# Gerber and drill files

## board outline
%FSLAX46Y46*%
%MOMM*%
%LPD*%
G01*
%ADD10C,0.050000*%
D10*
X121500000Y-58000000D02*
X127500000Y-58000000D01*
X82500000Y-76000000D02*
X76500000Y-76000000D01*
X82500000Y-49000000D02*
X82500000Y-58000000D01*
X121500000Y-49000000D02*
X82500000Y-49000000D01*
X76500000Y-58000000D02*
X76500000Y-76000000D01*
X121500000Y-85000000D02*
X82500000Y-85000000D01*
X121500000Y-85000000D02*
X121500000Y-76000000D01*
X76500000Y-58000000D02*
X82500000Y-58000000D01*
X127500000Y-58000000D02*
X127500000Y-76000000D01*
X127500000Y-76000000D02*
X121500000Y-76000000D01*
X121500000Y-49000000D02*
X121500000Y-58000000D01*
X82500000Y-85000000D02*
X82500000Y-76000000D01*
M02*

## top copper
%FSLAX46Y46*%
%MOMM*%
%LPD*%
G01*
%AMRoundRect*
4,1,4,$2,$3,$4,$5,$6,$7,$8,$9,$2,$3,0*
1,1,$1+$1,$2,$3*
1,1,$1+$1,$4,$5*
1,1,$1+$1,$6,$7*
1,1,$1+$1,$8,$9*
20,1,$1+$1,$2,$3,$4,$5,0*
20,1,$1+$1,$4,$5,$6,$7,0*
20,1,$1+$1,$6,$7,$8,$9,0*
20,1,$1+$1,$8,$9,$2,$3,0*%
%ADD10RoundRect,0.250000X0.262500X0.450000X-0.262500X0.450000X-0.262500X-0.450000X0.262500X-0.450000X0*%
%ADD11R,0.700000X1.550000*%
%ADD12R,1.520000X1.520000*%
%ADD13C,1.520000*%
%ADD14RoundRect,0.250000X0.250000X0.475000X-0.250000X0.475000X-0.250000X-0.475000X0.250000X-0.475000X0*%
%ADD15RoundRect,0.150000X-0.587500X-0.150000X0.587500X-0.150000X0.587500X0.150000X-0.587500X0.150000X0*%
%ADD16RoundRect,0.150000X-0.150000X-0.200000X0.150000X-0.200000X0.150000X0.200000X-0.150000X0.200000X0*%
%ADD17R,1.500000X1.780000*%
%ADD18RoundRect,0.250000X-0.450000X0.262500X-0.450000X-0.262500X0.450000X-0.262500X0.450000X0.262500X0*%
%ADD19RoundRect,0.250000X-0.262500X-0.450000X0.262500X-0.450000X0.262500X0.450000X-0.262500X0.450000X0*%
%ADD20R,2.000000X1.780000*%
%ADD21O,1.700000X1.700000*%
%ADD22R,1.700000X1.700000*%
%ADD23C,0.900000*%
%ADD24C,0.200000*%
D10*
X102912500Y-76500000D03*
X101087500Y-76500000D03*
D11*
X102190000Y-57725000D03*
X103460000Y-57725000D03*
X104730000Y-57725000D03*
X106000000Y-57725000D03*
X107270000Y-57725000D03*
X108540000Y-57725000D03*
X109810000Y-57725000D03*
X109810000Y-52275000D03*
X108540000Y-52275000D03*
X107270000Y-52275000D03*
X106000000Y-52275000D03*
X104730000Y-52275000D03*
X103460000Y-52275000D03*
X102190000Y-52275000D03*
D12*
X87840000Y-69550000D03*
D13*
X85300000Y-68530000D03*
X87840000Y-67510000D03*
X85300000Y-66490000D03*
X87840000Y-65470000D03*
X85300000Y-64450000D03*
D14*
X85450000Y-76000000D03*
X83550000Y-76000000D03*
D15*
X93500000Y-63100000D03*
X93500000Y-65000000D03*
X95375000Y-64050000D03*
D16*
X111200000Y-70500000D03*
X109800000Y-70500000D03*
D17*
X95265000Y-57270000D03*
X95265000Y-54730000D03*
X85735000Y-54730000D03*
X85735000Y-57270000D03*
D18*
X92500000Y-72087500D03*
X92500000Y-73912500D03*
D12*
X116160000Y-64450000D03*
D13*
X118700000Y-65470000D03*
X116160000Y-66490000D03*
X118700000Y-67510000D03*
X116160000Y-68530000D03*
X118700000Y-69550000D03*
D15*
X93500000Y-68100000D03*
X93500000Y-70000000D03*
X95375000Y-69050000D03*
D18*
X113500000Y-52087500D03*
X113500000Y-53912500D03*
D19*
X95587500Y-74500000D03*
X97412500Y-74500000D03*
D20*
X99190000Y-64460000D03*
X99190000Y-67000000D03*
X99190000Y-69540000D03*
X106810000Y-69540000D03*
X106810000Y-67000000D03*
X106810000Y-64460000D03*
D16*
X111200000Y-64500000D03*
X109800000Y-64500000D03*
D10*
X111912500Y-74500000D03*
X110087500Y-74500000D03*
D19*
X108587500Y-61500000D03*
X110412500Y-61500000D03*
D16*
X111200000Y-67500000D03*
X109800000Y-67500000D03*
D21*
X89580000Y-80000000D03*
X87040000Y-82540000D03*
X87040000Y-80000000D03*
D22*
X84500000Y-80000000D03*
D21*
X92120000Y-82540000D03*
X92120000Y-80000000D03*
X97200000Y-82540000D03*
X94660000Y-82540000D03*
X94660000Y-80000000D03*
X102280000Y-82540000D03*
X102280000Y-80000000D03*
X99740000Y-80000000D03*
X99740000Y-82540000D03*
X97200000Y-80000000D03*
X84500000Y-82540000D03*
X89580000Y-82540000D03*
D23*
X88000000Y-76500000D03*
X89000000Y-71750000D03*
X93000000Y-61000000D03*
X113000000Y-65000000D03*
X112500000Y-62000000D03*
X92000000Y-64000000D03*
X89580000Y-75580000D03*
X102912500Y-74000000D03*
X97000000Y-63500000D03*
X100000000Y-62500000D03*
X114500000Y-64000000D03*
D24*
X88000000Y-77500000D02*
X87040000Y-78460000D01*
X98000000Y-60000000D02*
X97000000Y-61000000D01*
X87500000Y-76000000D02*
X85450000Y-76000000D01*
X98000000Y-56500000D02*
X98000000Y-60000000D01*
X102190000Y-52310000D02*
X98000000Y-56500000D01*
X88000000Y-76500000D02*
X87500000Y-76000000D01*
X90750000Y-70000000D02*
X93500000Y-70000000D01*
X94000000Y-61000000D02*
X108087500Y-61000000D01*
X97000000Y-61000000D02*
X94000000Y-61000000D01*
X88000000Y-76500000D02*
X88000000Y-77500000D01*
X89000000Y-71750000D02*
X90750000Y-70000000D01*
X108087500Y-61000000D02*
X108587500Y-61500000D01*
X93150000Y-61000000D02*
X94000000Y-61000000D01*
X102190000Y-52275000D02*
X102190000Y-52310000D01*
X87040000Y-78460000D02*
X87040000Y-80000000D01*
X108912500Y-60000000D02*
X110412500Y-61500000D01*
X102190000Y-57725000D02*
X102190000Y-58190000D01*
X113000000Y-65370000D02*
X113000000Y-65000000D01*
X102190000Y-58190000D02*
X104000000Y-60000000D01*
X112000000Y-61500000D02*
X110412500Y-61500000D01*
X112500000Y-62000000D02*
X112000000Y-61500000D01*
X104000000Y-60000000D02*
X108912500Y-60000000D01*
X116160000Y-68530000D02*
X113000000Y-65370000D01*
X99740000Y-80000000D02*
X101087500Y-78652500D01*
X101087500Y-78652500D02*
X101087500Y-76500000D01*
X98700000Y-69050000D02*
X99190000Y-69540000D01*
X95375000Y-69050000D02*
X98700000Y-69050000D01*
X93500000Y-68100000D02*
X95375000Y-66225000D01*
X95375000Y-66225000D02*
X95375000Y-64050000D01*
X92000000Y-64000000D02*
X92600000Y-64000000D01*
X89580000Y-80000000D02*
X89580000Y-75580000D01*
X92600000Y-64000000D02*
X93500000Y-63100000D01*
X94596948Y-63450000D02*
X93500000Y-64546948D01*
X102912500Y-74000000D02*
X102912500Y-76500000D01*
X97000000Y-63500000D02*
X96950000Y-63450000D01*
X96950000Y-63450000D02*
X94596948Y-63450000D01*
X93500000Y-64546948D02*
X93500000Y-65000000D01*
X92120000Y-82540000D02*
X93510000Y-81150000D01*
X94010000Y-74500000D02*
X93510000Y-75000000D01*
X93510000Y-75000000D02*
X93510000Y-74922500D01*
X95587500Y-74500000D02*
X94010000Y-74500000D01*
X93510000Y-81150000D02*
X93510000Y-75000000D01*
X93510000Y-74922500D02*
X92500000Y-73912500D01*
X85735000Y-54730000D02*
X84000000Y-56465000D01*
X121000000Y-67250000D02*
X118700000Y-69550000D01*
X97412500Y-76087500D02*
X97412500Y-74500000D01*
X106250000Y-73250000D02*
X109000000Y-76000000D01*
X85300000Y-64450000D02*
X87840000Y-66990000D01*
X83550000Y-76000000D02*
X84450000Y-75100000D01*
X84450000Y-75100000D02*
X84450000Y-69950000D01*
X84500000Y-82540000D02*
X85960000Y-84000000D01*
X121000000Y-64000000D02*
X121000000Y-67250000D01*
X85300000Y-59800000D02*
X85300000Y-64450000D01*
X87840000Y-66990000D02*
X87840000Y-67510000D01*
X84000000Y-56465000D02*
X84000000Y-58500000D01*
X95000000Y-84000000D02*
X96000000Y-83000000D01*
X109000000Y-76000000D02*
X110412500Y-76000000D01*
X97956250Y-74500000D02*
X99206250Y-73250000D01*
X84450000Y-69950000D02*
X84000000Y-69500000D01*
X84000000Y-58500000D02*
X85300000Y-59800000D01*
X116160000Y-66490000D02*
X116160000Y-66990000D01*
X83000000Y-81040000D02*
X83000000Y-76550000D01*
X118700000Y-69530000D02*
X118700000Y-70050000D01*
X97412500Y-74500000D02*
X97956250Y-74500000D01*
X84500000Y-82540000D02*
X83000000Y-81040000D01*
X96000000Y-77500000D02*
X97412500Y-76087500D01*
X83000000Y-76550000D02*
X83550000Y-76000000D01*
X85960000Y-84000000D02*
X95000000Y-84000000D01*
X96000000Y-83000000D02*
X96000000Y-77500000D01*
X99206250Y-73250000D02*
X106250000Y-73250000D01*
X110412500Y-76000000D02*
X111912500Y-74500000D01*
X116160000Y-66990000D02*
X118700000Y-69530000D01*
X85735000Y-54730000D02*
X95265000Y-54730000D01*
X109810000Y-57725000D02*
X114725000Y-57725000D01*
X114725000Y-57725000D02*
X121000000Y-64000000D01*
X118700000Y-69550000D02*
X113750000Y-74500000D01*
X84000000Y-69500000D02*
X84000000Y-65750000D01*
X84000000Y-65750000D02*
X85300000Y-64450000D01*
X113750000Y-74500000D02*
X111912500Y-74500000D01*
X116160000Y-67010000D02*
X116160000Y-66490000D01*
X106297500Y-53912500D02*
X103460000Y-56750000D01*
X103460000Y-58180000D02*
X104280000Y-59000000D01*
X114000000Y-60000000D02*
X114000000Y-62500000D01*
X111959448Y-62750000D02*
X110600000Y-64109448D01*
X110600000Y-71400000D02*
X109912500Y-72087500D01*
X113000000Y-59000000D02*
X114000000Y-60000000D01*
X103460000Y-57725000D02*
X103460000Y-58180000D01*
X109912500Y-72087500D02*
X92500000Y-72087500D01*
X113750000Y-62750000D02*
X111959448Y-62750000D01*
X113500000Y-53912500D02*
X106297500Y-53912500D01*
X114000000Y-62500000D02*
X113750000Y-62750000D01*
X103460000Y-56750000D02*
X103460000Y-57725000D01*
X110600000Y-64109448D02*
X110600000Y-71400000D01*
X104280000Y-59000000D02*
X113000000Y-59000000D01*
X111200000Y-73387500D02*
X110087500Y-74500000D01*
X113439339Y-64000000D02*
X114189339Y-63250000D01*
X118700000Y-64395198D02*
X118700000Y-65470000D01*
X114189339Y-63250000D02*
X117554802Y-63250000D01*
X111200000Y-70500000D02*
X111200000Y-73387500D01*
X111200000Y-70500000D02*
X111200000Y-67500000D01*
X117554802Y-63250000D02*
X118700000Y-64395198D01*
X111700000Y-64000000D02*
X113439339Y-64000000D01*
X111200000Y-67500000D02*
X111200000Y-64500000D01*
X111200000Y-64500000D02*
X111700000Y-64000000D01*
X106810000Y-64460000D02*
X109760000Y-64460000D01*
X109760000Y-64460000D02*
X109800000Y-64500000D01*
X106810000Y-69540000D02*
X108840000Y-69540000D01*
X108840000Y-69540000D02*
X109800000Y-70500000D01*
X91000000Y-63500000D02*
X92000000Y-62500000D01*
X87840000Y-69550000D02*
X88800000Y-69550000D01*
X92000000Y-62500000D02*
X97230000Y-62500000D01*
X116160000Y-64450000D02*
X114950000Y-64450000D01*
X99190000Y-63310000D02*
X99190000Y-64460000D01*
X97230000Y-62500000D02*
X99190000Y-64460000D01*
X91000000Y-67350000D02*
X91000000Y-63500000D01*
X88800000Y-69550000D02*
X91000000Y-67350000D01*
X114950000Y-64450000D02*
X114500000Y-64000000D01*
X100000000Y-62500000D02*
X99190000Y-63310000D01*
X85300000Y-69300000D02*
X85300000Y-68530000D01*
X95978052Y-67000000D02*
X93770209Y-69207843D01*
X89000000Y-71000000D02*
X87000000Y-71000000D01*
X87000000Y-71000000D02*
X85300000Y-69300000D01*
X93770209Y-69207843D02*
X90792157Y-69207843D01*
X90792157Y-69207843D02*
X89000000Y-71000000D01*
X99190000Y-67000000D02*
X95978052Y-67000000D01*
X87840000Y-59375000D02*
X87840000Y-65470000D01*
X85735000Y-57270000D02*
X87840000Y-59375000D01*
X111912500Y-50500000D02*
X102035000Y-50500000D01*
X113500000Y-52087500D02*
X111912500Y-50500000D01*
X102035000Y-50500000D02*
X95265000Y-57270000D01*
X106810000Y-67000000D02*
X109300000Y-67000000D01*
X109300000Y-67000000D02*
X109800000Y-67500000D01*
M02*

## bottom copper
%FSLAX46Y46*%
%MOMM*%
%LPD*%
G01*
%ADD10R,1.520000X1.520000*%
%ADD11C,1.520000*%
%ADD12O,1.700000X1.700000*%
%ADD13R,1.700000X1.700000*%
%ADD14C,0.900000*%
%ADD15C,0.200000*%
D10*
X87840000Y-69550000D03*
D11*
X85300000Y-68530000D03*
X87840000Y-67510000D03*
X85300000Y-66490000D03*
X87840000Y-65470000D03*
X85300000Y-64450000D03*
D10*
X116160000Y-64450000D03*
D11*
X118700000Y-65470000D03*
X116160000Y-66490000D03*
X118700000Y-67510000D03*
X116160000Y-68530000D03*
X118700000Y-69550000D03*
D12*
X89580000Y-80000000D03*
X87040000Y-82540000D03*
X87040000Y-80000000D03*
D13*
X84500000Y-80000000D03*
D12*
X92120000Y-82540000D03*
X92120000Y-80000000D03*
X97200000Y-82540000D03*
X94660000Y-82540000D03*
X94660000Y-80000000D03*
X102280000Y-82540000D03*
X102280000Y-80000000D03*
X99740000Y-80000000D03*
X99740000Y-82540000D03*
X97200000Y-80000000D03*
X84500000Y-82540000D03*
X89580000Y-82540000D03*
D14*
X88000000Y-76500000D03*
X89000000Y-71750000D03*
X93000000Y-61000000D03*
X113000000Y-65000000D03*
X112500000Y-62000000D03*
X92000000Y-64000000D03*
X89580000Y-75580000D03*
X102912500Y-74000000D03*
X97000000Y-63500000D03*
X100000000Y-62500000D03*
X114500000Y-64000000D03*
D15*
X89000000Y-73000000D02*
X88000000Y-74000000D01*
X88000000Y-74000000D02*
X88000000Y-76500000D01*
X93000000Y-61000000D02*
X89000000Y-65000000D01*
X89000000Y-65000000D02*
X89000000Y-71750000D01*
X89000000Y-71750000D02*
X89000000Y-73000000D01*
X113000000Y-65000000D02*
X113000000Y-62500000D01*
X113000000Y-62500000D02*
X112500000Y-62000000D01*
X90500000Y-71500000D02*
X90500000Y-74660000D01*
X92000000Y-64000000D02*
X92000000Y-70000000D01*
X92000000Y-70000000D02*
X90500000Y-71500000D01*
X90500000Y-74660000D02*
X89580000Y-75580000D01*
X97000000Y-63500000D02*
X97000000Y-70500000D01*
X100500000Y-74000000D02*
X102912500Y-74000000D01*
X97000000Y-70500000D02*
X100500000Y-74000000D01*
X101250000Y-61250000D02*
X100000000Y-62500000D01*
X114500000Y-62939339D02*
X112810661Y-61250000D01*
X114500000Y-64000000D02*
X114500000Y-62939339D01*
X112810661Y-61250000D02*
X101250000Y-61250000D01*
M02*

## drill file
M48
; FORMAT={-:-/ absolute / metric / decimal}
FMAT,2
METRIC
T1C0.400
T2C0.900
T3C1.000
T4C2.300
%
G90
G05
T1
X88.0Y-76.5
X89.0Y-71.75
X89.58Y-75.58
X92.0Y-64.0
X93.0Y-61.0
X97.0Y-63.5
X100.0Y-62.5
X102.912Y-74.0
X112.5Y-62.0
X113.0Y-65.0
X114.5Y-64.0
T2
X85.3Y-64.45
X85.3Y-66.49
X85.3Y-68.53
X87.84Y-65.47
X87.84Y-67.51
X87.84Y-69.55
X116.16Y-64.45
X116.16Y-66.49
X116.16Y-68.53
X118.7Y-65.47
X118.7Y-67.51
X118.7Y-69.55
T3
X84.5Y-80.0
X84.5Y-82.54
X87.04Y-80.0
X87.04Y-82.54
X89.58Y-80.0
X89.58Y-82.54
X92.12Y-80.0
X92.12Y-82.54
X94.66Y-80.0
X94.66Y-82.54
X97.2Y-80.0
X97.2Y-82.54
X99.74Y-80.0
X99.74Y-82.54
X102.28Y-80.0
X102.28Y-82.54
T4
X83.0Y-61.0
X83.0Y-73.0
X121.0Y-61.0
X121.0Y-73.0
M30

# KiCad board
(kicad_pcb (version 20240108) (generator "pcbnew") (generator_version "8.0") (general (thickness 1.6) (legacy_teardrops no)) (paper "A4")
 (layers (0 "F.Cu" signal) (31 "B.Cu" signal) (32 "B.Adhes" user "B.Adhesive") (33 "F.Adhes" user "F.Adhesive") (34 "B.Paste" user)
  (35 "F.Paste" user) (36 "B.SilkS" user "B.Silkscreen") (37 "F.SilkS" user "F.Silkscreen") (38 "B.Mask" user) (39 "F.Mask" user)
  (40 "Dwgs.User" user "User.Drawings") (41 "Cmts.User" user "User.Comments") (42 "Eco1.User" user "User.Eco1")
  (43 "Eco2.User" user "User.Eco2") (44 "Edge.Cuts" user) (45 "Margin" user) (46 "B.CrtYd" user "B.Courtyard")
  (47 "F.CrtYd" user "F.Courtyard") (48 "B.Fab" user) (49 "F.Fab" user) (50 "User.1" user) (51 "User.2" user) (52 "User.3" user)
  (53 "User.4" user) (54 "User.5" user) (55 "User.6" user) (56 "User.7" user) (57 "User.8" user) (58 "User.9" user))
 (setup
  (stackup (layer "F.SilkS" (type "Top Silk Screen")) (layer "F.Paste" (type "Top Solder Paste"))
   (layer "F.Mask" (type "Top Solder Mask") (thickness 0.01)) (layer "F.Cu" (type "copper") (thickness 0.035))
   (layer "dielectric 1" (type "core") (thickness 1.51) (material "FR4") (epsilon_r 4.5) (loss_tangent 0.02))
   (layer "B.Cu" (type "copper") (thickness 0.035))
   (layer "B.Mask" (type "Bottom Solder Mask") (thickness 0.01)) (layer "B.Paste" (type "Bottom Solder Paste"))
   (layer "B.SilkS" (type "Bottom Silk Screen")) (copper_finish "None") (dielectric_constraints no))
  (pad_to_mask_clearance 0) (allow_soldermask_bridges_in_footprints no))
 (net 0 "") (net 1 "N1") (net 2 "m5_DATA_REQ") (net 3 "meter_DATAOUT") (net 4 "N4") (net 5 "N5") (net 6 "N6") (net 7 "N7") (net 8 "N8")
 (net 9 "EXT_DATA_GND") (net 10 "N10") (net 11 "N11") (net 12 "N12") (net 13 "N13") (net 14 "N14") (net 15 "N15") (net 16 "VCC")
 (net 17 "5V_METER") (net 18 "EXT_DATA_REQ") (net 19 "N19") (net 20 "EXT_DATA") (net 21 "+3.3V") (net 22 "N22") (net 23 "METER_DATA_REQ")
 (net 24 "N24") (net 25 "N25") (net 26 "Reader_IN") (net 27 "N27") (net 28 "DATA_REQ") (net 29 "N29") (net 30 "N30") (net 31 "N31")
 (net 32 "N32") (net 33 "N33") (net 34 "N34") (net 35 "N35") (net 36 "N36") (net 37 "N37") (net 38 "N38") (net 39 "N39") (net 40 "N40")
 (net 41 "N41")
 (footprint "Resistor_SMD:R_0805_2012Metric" (layer "F.Cu") (at 102 76.5 180)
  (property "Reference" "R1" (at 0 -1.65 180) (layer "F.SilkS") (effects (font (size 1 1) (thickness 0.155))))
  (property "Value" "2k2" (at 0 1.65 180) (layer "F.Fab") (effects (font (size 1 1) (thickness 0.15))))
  (pad "1" smd roundrect (at -0.9125 0 180) (size 1.025 1.4) (layers "F.Cu" "F.Paste" "F.Mask") (roundrect_rratio 0.243902) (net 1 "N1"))
  (pad "2" smd roundrect (at 0.9125 0 180) (size 1.025 1.4) (layers "F.Cu" "F.Paste" "F.Mask") (roundrect_rratio 0.243902)
   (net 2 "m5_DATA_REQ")))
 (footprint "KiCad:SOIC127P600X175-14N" (layer "F.Cu") (at 106 55 90)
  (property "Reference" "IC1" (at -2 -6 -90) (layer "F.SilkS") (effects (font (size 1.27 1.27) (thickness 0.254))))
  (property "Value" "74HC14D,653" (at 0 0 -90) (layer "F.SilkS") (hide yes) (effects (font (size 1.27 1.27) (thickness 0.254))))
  (pad "1" smd rect (at -2.725 -3.81 180) (size 0.7 1.55) (layers "F.Cu" "F.Paste" "F.Mask") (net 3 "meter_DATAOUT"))
  (pad "2" smd rect (at -2.725 -2.54 180) (size 0.7 1.55) (layers "F.Cu" "F.Paste" "F.Mask") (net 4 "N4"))
  (pad "3" smd rect (at -2.725 -1.27 180) (size 0.7 1.55) (layers "F.Cu" "F.Paste" "F.Mask") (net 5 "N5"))
  (pad "4" smd rect (at -2.725 0 180) (size 0.7 1.55) (layers "F.Cu" "F.Paste" "F.Mask") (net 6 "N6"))
  (pad "5" smd rect (at -2.725 1.27 180) (size 0.7 1.55) (layers "F.Cu" "F.Paste" "F.Mask") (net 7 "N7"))
  (pad "6" smd rect (at -2.725 2.54 180) (size 0.7 1.55) (layers "F.Cu" "F.Paste" "F.Mask") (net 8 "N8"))
  (pad "7" smd rect (at -2.725 3.81 180) (size 0.7 1.55) (layers "F.Cu" "F.Paste" "F.Mask") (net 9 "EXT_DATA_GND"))
  (pad "8" smd rect (at 2.725 3.81 180) (size 0.7 1.55) (layers "F.Cu" "F.Paste" "F.Mask") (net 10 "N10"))
  (pad "9" smd rect (at 2.725 2.54 180) (size 0.7 1.55) (layers "F.Cu" "F.Paste" "F.Mask") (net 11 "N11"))
  (pad "10" smd rect (at 2.725 1.27 180) (size 0.7 1.55) (layers "F.Cu" "F.Paste" "F.Mask") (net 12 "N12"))
  (pad "11" smd rect (at 2.725 0 180) (size 0.7 1.55) (layers "F.Cu" "F.Paste" "F.Mask") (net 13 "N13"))
  (pad "12" smd rect (at 2.725 -1.27 180) (size 0.7 1.55) (layers "F.Cu" "F.Paste" "F.Mask") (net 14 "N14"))
  (pad "13" smd rect (at 2.725 -2.54 180) (size 0.7 1.55) (layers "F.Cu" "F.Paste" "F.Mask") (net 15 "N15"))
  (pad "14" smd rect (at 2.725 -3.81 180) (size 0.7 1.55) (layers "F.Cu" "F.Paste" "F.Mask") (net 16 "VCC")))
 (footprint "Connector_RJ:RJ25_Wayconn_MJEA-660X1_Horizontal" (layer "F.Cu") (at 87.84 69.55 -90)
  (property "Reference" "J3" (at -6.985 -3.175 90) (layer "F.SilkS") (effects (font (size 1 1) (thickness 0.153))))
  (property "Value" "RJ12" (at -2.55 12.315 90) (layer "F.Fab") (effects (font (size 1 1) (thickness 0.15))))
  (pad "" np_thru_hole circle (at -8.55 4.84 270) (size 2.3 2.3) (drill 2.3) (layers "*.Cu" "*.Mask"))
  (pad "" np_thru_hole circle (at 3.45 4.84 270) (size 2.3 2.3) (drill 2.3) (layers "*.Cu" "*.Mask"))
  (pad "1" thru_hole rect (at 0 0 270) (size 1.52 1.52) (drill 0.9) (layers "*.Cu" "*.Mask") (remove_unused_layers no) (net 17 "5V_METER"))
  (pad "2" thru_hole circle (at -1.02 2.54 270) (size 1.52 1.52) (drill 0.9) (layers "*.Cu" "*.Mask") (remove_unused_layers no)
   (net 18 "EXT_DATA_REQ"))
  (pad "3" thru_hole circle (at -2.04 0 270) (size 1.52 1.52) (drill 0.9) (layers "*.Cu" "*.Mask") (remove_unused_layers no)
   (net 9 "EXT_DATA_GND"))
  (pad "4" thru_hole circle (at -3.06 2.54 270) (size 1.52 1.52) (drill 0.9) (layers "*.Cu" "*.Mask") (remove_unused_layers no)
   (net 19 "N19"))
  (pad "5" thru_hole circle (at -4.08 0 270) (size 1.52 1.52) (drill 0.9) (layers "*.Cu" "*.Mask") (remove_unused_layers no)
   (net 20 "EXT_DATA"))
  (pad "6" thru_hole circle (at -5.1 2.54 270) (size 1.52 1.52) (drill 0.9) (layers "*.Cu" "*.Mask") (remove_unused_layers no)
   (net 9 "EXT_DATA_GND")))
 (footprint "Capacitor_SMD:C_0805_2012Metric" (layer "F.Cu") (at 84.5 76 180)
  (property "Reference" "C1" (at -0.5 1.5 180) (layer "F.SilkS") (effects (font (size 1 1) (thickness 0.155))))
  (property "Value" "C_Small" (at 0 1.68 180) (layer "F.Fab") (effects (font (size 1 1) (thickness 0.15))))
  (pad "1" smd roundrect (at -0.95 0 180) (size 1 1.45) (layers "F.Cu" "F.Paste" "F.Mask") (roundrect_rratio 0.25) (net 16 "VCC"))
  (pad "2" smd roundrect (at 0.95 0 180) (size 1 1.45) (layers "F.Cu" "F.Paste" "F.Mask") (roundrect_rratio 0.25) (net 9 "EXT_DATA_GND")))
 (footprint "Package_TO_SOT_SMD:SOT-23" (layer "F.Cu") (at 94.4375 64.05)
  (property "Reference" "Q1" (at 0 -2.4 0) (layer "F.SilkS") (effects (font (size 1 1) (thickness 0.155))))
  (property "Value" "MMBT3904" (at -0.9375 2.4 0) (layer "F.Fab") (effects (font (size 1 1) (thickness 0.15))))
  (pad "1" smd roundrect (at -0.9375 -0.95) (size 1.475 0.6) (layers "F.Cu" "F.Paste" "F.Mask") (roundrect_rratio 0.25) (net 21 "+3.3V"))
  (pad "2" smd roundrect (at -0.9375 0.95) (size 1.475 0.6) (layers "F.Cu" "F.Paste" "F.Mask") (roundrect_rratio 0.25) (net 1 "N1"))
  (pad "3" smd roundrect (at 0.9375 0) (size 1.475 0.6) (layers "F.Cu" "F.Paste" "F.Mask") (roundrect_rratio 0.25) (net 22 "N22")))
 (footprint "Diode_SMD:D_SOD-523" (layer "F.Cu") (at 110.5 70.5 180)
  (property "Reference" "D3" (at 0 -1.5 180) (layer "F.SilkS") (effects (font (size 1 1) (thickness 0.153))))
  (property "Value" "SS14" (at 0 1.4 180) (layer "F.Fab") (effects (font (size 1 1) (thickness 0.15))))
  (pad "1" smd roundrect (at -0.7 0) (size 0.6 0.7) (layers "F.Cu" "F.Paste" "F.Mask") (roundrect_rratio 0.25) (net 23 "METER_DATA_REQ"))
  (pad "2" smd roundrect (at 0.7 0) (size 0.6 0.7) (layers "F.Cu" "F.Paste" "F.Mask") (roundrect_rratio 0.25) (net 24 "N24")))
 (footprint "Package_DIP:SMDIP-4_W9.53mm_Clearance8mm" (layer "F.Cu") (at 90.5 56 180)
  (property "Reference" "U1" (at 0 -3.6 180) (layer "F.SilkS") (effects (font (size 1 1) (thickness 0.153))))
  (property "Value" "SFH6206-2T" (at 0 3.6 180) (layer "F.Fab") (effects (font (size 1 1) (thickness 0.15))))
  (pad "1" smd rect (at -4.765 -1.27 180) (size 1.5 1.78) (layers "F.Cu" "F.Paste" "F.Mask") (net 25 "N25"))
  (pad "2" smd rect (at -4.765 1.27 180) (size 1.5 1.78) (layers "F.Cu" "F.Paste" "F.Mask") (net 9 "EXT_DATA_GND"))
  (pad "3" smd rect (at 4.765 1.27 180) (size 1.5 1.78) (layers "F.Cu" "F.Paste" "F.Mask") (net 9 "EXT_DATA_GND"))
  (pad "4" smd rect (at 4.765 -1.27 180) (size 1.5 1.78) (layers "F.Cu" "F.Paste" "F.Mask") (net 20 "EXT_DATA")))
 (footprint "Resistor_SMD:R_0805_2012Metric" (layer "F.Cu") (at 92.5 73 -90)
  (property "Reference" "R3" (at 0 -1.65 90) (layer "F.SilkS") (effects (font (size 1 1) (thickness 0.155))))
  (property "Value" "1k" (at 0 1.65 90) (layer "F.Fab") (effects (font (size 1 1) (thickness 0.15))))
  (pad "1" smd roundrect (at -0.9125 0 270) (size 1.025 1.4) (layers "F.Cu" "F.Paste" "F.Mask") (roundrect_rratio 0.243902) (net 4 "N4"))
  (pad "2" smd roundrect (at 0.9125 0 270) (size 1.025 1.4) (layers "F.Cu" "F.Paste" "F.Mask") (roundrect_rratio 0.243902)
   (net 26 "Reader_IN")))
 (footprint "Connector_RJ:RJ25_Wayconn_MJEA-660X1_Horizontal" (layer "F.Cu") (at 116.16 64.45 90)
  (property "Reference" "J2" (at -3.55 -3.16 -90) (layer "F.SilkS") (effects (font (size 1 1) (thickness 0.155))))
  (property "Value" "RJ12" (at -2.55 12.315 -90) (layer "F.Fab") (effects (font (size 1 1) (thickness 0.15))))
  (pad "" np_thru_hole circle (at -8.55 4.84 90) (size 2.3 2.3) (drill 2.3) (layers "*.Cu" "*.Mask"))
  (pad "" np_thru_hole circle (at 3.45 4.84 90) (size 2.3 2.3) (drill 2.3) (layers "*.Cu" "*.Mask"))
  (pad "1" thru_hole rect (at 0 0 90) (size 1.52 1.52) (drill 0.9) (layers "*.Cu" "*.Mask") (remove_unused_layers no) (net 17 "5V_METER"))
  (pad "2" thru_hole circle (at -1.02 2.54 90) (size 1.52 1.52) (drill 0.9) (layers "*.Cu" "*.Mask") (remove_unused_layers no)
   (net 23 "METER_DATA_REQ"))
  (pad "3" thru_hole circle (at -2.04 0 90) (size 1.52 1.52) (drill 0.9) (layers "*.Cu" "*.Mask") (remove_unused_layers no)
   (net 9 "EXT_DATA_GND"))
  (pad "4" thru_hole circle (at -3.06 2.54 90) (size 1.52 1.52) (drill 0.9) (layers "*.Cu" "*.Mask") (remove_unused_layers no)
   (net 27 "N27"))
  (pad "5" thru_hole circle (at -4.08 0 90) (size 1.52 1.52) (drill 0.9) (layers "*.Cu" "*.Mask") (remove_unused_layers no)
   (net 3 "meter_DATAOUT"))
  (pad "6" thru_hole circle (at -5.1 2.54 90) (size 1.52 1.52) (drill 0.9) (layers "*.Cu" "*.Mask") (remove_unused_layers no)
   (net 9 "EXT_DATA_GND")))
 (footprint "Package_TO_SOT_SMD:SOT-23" (layer "F.Cu") (at 94.4375 69.05)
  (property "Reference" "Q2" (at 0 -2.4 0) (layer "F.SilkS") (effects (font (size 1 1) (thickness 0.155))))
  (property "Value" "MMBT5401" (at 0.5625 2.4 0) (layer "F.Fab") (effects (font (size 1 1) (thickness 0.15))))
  (pad "1" smd roundrect (at -0.9375 -0.95) (size 1.475 0.6) (layers "F.Cu" "F.Paste" "F.Mask") (roundrect_rratio 0.25) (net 22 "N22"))
  (pad "2" smd roundrect (at -0.9375 0.95) (size 1.475 0.6) (layers "F.Cu" "F.Paste" "F.Mask") (roundrect_rratio 0.25) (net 16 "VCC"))
  (pad "3" smd roundrect (at 0.9375 0) (size 1.475 0.6) (layers "F.Cu" "F.Paste" "F.Mask") (roundrect_rratio 0.25) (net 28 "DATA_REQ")))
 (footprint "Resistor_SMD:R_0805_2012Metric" (layer "F.Cu") (at 113.5 53 -90)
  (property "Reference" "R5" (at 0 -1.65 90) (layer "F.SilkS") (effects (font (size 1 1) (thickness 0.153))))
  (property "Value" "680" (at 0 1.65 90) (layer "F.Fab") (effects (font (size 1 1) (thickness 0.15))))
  (pad "1" smd roundrect (at -0.9125 0 270) (size 1.025 1.4) (layers "F.Cu" "F.Paste" "F.Mask") (roundrect_rratio 0.243902) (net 25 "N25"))
  (pad "2" smd roundrect (at 0.9125 0 270) (size 1.025 1.4) (layers "F.Cu" "F.Paste" "F.Mask") (roundrect_rratio 0.243902) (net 4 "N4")))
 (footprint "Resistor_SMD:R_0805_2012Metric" (layer "F.Cu") (at 96.5 74.5)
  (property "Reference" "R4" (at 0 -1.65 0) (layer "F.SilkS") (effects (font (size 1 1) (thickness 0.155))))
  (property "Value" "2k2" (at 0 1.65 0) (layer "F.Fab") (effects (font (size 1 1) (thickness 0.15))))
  (pad "1" smd roundrect (at -0.9125 0) (size 1.025 1.4) (layers "F.Cu" "F.Paste" "F.Mask") (roundrect_rratio 0.243902) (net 26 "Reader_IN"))
  (pad "2" smd roundrect (at 0.9125 0) (size 1.025 1.4) (layers "F.Cu" "F.Paste" "F.Mask") (roundrect_rratio 0.243902)
   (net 9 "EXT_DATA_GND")))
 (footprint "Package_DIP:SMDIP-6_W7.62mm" (layer "F.Cu") (at 103 67)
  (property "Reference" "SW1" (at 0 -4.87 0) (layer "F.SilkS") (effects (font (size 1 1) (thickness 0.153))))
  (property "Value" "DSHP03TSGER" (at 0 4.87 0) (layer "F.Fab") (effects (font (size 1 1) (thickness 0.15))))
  (pad "1" smd rect (at -3.81 -2.54) (size 2 1.78) (layers "F.Cu" "F.Paste" "F.Mask") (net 17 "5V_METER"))
  (pad "2" smd rect (at -3.81 0) (size 2 1.78) (layers "F.Cu" "F.Paste" "F.Mask") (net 18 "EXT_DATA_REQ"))
  (pad "3" smd rect (at -3.81 2.54) (size 2 1.78) (layers "F.Cu" "F.Paste" "F.Mask") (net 28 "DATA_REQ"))
  (pad "4" smd rect (at 3.81 2.54) (size 2 1.78) (layers "F.Cu" "F.Paste" "F.Mask") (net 24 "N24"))
  (pad "5" smd rect (at 3.81 0) (size 2 1.78) (layers "F.Cu" "F.Paste" "F.Mask") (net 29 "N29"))
  (pad "6" smd rect (at 3.81 -2.54) (size 2 1.78) (layers "F.Cu" "F.Paste" "F.Mask") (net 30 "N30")))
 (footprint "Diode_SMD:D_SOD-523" (layer "F.Cu") (at 110.5 64.5 180)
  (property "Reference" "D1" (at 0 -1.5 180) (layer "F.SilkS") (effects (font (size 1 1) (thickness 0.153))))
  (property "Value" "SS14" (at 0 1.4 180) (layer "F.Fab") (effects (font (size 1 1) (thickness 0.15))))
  (pad "1" smd roundrect (at -0.7 0) (size 0.6 0.7) (layers "F.Cu" "F.Paste" "F.Mask") (roundrect_rratio 0.25) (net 23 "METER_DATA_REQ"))
  (pad "2" smd roundrect (at 0.7 0) (size 0.6 0.7) (layers "F.Cu" "F.Paste" "F.Mask") (roundrect_rratio 0.25) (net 30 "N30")))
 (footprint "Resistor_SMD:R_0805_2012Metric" (layer "F.Cu") (at 111 74.5 180)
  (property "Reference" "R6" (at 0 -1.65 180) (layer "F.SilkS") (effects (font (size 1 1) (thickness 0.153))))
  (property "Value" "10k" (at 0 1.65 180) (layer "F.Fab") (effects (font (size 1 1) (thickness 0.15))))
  (pad "1" smd roundrect (at -0.9125 0 180) (size 1.025 1.4) (layers "F.Cu" "F.Paste" "F.Mask") (roundrect_rratio 0.243902)
   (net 9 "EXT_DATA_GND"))
  (pad "2" smd roundrect (at 0.9125 0 180) (size 1.025 1.4) (layers "F.Cu" "F.Paste" "F.Mask") (roundrect_rratio 0.243902)
   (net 23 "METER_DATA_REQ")))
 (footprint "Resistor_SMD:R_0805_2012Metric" (layer "F.Cu") (at 109.5 61.5)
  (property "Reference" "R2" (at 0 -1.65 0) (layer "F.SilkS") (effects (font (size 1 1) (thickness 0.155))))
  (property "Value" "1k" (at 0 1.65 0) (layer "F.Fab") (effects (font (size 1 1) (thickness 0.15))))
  (pad "1" smd roundrect (at -0.9125 0) (size 1.025 1.4) (layers "F.Cu" "F.Paste" "F.Mask") (roundrect_rratio 0.243902) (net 16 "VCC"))
  (pad "2" smd roundrect (at 0.9125 0) (size 1.025 1.4) (layers "F.Cu" "F.Paste" "F.Mask") (roundrect_rratio 0.243902)
   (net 3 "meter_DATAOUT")))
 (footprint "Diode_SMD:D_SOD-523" (layer "F.Cu") (at 110.5 67.5 180)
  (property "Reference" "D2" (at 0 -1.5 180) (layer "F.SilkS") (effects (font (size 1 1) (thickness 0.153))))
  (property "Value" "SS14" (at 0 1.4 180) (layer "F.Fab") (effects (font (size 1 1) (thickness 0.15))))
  (pad "1" smd roundrect (at -0.7 0) (size 0.6 0.7) (layers "F.Cu" "F.Paste" "F.Mask") (roundrect_rratio 0.25) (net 23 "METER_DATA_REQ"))
  (pad "2" smd roundrect (at 0.7 0) (size 0.6 0.7) (layers "F.Cu" "F.Paste" "F.Mask") (roundrect_rratio 0.25) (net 29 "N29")))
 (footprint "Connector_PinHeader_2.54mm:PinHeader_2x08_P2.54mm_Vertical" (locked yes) (layer "B.Cu") (at 84.5 80 -90)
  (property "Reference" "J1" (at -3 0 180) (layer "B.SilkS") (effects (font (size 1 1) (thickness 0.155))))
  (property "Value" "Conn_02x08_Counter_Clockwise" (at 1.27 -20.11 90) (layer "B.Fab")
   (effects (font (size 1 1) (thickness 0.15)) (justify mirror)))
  (pad "3V3" thru_hole oval (at 0 -5.08 270) (size 1.7 1.7) (drill 1) (layers "*.Cu" "*.Mask") (remove_unused_layers no) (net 21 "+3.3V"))
  (pad "5VIN" thru_hole oval (at 2.54 -2.54 270) (size 1.7 1.7) (drill 1) (layers "*.Cu" "*.Mask") (remove_unused_layers no) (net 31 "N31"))
  (pad "5VOUT" thru_hole oval (at 0 -2.54 270) (size 1.7 1.7) (drill 1) (layers "*.Cu" "*.Mask") (remove_unused_layers no) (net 16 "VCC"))
  (pad "BAT" thru_hole rect (at 0 0 270) (size 1.7 1.7) (drill 1) (layers "*.Cu" "*.Mask") (remove_unused_layers no) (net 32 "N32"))
  (pad "G13" thru_hole oval (at 2.54 -7.62 270) (size 1.7 1.7) (drill 1) (layers "*.Cu" "*.Mask") (remove_unused_layers no)
   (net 26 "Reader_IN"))
  (pad "G14" thru_hole oval (at 0 -7.62 270) (size 1.7 1.7) (drill 1) (layers "*.Cu" "*.Mask") (remove_unused_layers no) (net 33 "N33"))
  (pad "G18" thru_hole oval (at 2.54 -12.7 270) (size 1.7 1.7) (drill 1) (layers "*.Cu" "*.Mask") (remove_unused_layers no) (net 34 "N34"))
  (pad "G21" thru_hole oval (at 2.54 -10.16 270) (size 1.7 1.7) (drill 1) (layers "*.Cu" "*.Mask") (remove_unused_layers no) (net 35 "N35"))
  (pad "G22" thru_hole oval (at 0 -10.16 270) (size 1.7 1.7) (drill 1) (layers "*.Cu" "*.Mask") (remove_unused_layers no) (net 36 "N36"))
  (pad "G23" thru_hole oval (at 2.54 -17.78 270) (size 1.7 1.7) (drill 1) (layers "*.Cu" "*.Mask") (remove_unused_layers no) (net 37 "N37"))
  (pad "G25" thru_hole oval (at 0 -17.78 270) (size 1.7 1.7) (drill 1) (layers "*.Cu" "*.Mask") (remove_unused_layers no) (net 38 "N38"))
  (pad "G26" thru_hole oval (at 0 -15.24 270) (size 1.7 1.7) (drill 1) (layers "*.Cu" "*.Mask") (remove_unused_layers no)
   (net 2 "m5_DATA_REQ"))
  (pad "G34" thru_hole oval (at 2.54 -15.24 270) (size 1.7 1.7) (drill 1) (layers "*.Cu" "*.Mask") (remove_unused_layers no) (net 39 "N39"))
  (pad "G36" thru_hole oval (at 0 -12.7 270) (size 1.7 1.7) (drill 1) (layers "*.Cu" "*.Mask") (remove_unused_layers no) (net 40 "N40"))
  (pad "GND" thru_hole oval (at 2.54 0 270) (size 1.7 1.7) (drill 1) (layers "*.Cu" "*.Mask") (remove_unused_layers no)
   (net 9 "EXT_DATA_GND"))
  (pad "RST" thru_hole oval (at 2.54 -5.08 270) (size 1.7 1.7) (drill 1) (layers "*.Cu" "*.Mask") (remove_unused_layers no) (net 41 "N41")))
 (gr_line (start 121.5 58) (end 127.5 58) (stroke (width 0.05) (type default)) (layer "Edge.Cuts"))
 (gr_line (start 82.5 76) (end 76.5 76) (stroke (width 0.05) (type default)) (layer "Edge.Cuts"))
 (gr_line (start 82.5 49) (end 82.5 58) (stroke (width 0.05) (type default)) (layer "Edge.Cuts"))
 (gr_line (start 121.5 49) (end 82.5 49) (stroke (width 0.05) (type default)) (layer "Edge.Cuts"))
 (gr_line (start 76.5 58) (end 76.5 76) (stroke (width 0.05) (type default)) (layer "Edge.Cuts"))
 (gr_line (start 121.5 85) (end 82.5 85) (stroke (width 0.05) (type default)) (layer "Edge.Cuts"))
 (gr_line (start 121.5 85) (end 121.5 76) (stroke (width 0.05) (type default)) (layer "Edge.Cuts"))
 (gr_line (start 76.5 58) (end 82.5 58) (stroke (width 0.05) (type default)) (layer "Edge.Cuts"))
 (gr_line (start 127.5 58) (end 127.5 76) (stroke (width 0.05) (type default)) (layer "Edge.Cuts"))
 (gr_line (start 127.5 76) (end 121.5 76) (stroke (width 0.05) (type default)) (layer "Edge.Cuts"))
 (gr_line (start 121.5 49) (end 121.5 58) (stroke (width 0.05) (type default)) (layer "Edge.Cuts"))
 (gr_line (start 82.5 85) (end 82.5 76) (stroke (width 0.05) (type default)) (layer "Edge.Cuts"))
 (segment (start 88 77.5) (end 87.04 78.46) (width 0.2) (layer "F.Cu") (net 16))
 (segment (start 98 60) (end 97 61) (width 0.2) (layer "F.Cu") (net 16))
 (segment (start 87.5 76) (end 85.45 76) (width 0.2) (layer "F.Cu") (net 16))
 (segment (start 98 56.5) (end 98 60) (width 0.2) (layer "F.Cu") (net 16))
 (segment (start 102.19 52.31) (end 98 56.5) (width 0.2) (layer "F.Cu") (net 16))
 (segment (start 88 76.5) (end 87.5 76) (width 0.2) (layer "F.Cu") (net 16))
 (segment (start 90.75 70) (end 93.5 70) (width 0.2) (layer "F.Cu") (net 16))
 (segment (start 94 61) (end 108.0875 61) (width 0.2) (layer "F.Cu") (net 16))
 (segment (start 97 61) (end 94 61) (width 0.2) (layer "F.Cu") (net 16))
 (segment (start 88 76.5) (end 88 77.5) (width 0.2) (layer "F.Cu") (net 16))
 (segment (start 89 71.75) (end 90.75 70) (width 0.2) (layer "F.Cu") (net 16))
 (segment (start 108.0875 61) (end 108.5875 61.5) (width 0.2) (layer "F.Cu") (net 16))
 (segment (start 93.15 61) (end 94 61) (width 0.2) (layer "F.Cu") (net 16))
 (segment (start 102.19 52.275) (end 102.19 52.31) (width 0.2) (layer "F.Cu") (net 16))
 (segment (start 87.04 78.46) (end 87.04 80) (width 0.2) (layer "F.Cu") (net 16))
 (via (at 88 76.5) (size 0.9) (drill 0.4) (layers "F.Cu" "B.Cu") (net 16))
 (via (at 89 71.75) (size 0.9) (drill 0.4) (layers "F.Cu" "B.Cu") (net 16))
 (via (at 93 61) (size 0.9) (drill 0.4) (layers "F.Cu" "B.Cu") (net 16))
 (segment (start 89 73) (end 88 74) (width 0.2) (layer "B.Cu") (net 16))
 (segment (start 88 74) (end 88 76.5) (width 0.2) (layer "B.Cu") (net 16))
 (segment (start 93 61) (end 89 65) (width 0.2) (layer "B.Cu") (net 16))
 (segment (start 89 65) (end 89 71.75) (width 0.2) (layer "B.Cu") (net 16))
 (segment (start 89 71.75) (end 89 73) (width 0.2) (layer "B.Cu") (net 16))
 (segment (start 108.9125 60) (end 110.4125 61.5) (width 0.2) (layer "F.Cu") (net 3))
 (segment (start 102.19 57.725) (end 102.19 58.19) (width 0.2) (layer "F.Cu") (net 3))
 (segment (start 113 65.37) (end 113 65) (width 0.2) (layer "F.Cu") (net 3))
 (segment (start 102.19 58.19) (end 104 60) (width 0.2) (layer "F.Cu") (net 3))
 (segment (start 112 61.5) (end 110.4125 61.5) (width 0.2) (layer "F.Cu") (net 3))
 (segment (start 112.5 62) (end 112 61.5) (width 0.2) (layer "F.Cu") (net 3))
 (segment (start 104 60) (end 108.9125 60) (width 0.2) (layer "F.Cu") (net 3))
 (segment (start 116.16 68.53) (end 113 65.37) (width 0.2) (layer "F.Cu") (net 3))
 (via (at 113 65) (size 0.9) (drill 0.4) (layers "F.Cu" "B.Cu") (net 3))
 (via (at 112.5 62) (size 0.9) (drill 0.4) (layers "F.Cu" "B.Cu") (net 3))
 (segment (start 113 65) (end 113 62.5) (width 0.2) (layer "B.Cu") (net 3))
 (segment (start 113 62.5) (end 112.5 62) (width 0.2) (layer "B.Cu") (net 3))
 (segment (start 99.74 80) (end 101.0875 78.6525) (width 0.2) (layer "F.Cu") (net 2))
 (segment (start 101.0875 78.6525) (end 101.0875 76.5) (width 0.2) (layer "F.Cu") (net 2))
 (segment (start 98.7 69.05) (end 99.19 69.54) (width 0.2) (layer "F.Cu") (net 28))
 (segment (start 95.375 69.05) (end 98.7 69.05) (width 0.2) (layer "F.Cu") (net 28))
 (segment (start 93.5 68.1) (end 95.375 66.225) (width 0.2) (layer "F.Cu") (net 22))
 (segment (start 95.375 66.225) (end 95.375 64.05) (width 0.2) (layer "F.Cu") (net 22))
 (segment (start 92 64) (end 92.6 64) (width 0.2) (layer "F.Cu") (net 21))
 (segment (start 89.58 80) (end 89.58 75.58) (width 0.2) (layer "F.Cu") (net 21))
 (segment (start 92.6 64) (end 93.5 63.1) (width 0.2) (layer "F.Cu") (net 21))
 (via (at 92 64) (size 0.9) (drill 0.4) (layers "F.Cu" "B.Cu") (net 21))
 (via (at 89.58 75.58) (size 0.9) (drill 0.4) (layers "F.Cu" "B.Cu") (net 21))
 (segment (start 90.5 71.5) (end 90.5 74.66) (width 0.2) (layer "B.Cu") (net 21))
 (segment (start 92 64) (end 92 70) (width 0.2) (layer "B.Cu") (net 21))
 (segment (start 92 70) (end 90.5 71.5) (width 0.2) (layer "B.Cu") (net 21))
 (segment (start 90.5 74.66) (end 89.58 75.58) (width 0.2) (layer "B.Cu") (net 21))
 (segment (start 94.596948 63.45) (end 93.5 64.546948) (width 0.2) (layer "F.Cu") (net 1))
 (segment (start 102.9125 74) (end 102.9125 76.5) (width 0.2) (layer "F.Cu") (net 1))
 (segment (start 97 63.5) (end 96.95 63.45) (width 0.2) (layer "F.Cu") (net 1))
 (segment (start 96.95 63.45) (end 94.596948 63.45) (width 0.2) (layer "F.Cu") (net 1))
 (segment (start 93.5 64.546948) (end 93.5 65) (width 0.2) (layer "F.Cu") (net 1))
 (via (at 102.9125 74) (size 0.9) (drill 0.4) (layers "F.Cu" "B.Cu") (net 1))
 (via (at 97 63.5) (size 0.9) (drill 0.4) (layers "F.Cu" "B.Cu") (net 1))
 (segment (start 97 63.5) (end 97 70.5) (width 0.2) (layer "B.Cu") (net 1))
 (segment (start 100.5 74) (end 102.9125 74) (width 0.2) (layer "B.Cu") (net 1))
 (segment (start 97 70.5) (end 100.5 74) (width 0.2) (layer "B.Cu") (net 1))
 (segment (start 92.12 82.54) (end 93.51 81.15) (width 0.2) (layer "F.Cu") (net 26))
 (segment (start 94.01 74.5) (end 93.51 75) (width 0.2) (layer "F.Cu") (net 26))
 (segment (start 93.51 75) (end 93.51 74.9225) (width 0.2) (layer "F.Cu") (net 26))
 (segment (start 95.5875 74.5) (end 94.01 74.5) (width 0.2) (layer "F.Cu") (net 26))
 (segment (start 93.51 81.15) (end 93.51 75) (width 0.2) (layer "F.Cu") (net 26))
 (segment (start 93.51 74.9225) (end 92.5 73.9125) (width 0.2) (layer "F.Cu") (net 26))
 (segment (start 85.735 54.73) (end 84 56.465) (width 0.2) (layer "F.Cu") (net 9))
 (segment (start 121 67.25) (end 118.7 69.55) (width 0.2) (layer "F.Cu") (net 9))
 (segment (start 97.4125 76.0875) (end 97.4125 74.5) (width 0.2) (layer "F.Cu") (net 9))
 (segment (start 106.25 73.25) (end 109 76) (width 0.2) (layer "F.Cu") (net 9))
 (segment (start 85.3 64.45) (end 87.84 66.99) (width 0.2) (layer "F.Cu") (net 9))
 (segment (start 83.55 76) (end 84.45 75.1) (width 0.2) (layer "F.Cu") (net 9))
 (segment (start 84.45 75.1) (end 84.45 69.95) (width 0.2) (layer "F.Cu") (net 9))
 (segment (start 84.5 82.54) (end 85.96 84) (width 0.2) (layer "F.Cu") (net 9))
 (segment (start 121 64) (end 121 67.25) (width 0.2) (layer "F.Cu") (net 9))
 (segment (start 85.3 59.8) (end 85.3 64.45) (width 0.2) (layer "F.Cu") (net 9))
 (segment (start 87.84 66.99) (end 87.84 67.51) (width 0.2) (layer "F.Cu") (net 9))
 (segment (start 84 56.465) (end 84 58.5) (width 0.2) (layer "F.Cu") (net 9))
 (segment (start 95 84) (end 96 83) (width 0.2) (layer "F.Cu") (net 9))
 (segment (start 109 76) (end 110.4125 76) (width 0.2) (layer "F.Cu") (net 9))
 (segment (start 97.95625 74.5) (end 99.20625 73.25) (width 0.2) (layer "F.Cu") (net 9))
 (segment (start 84.45 69.95) (end 84 69.5) (width 0.2) (layer "F.Cu") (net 9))
 (segment (start 84 58.5) (end 85.3 59.8) (width 0.2) (layer "F.Cu") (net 9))
 (segment (start 116.16 66.49) (end 116.16 66.99) (width 0.2) (layer "F.Cu") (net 9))
 (segment (start 83 81.04) (end 83 76.55) (width 0.2) (layer "F.Cu") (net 9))
 (segment (start 118.7 69.53) (end 118.7 70.05) (width 0.2) (layer "F.Cu") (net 9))
 (segment (start 97.4125 74.5) (end 97.95625 74.5) (width 0.2) (layer "F.Cu") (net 9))
 (segment (start 84.5 82.54) (end 83 81.04) (width 0.2) (layer "F.Cu") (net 9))
 (segment (start 96 77.5) (end 97.4125 76.0875) (width 0.2) (layer "F.Cu") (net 9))
 (segment (start 83 76.55) (end 83.55 76) (width 0.2) (layer "F.Cu") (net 9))
 (segment (start 85.96 84) (end 95 84) (width 0.2) (layer "F.Cu") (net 9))
 (segment (start 96 83) (end 96 77.5) (width 0.2) (layer "F.Cu") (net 9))
 (segment (start 99.20625 73.25) (end 106.25 73.25) (width 0.2) (layer "F.Cu") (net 9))
 (segment (start 110.4125 76) (end 111.9125 74.5) (width 0.2) (layer "F.Cu") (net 9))
 (segment (start 116.16 66.99) (end 118.7 69.53) (width 0.2) (layer "F.Cu") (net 9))
 (segment (start 85.735 54.73) (end 95.265 54.73) (width 0.2) (layer "F.Cu") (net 9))
 (segment (start 109.81 57.725) (end 114.725 57.725) (width 0.2) (layer "F.Cu") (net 9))
 (segment (start 114.725 57.725) (end 121 64) (width 0.2) (layer "F.Cu") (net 9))
 (segment (start 118.7 69.55) (end 113.75 74.5) (width 0.2) (layer "F.Cu") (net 9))
 (segment (start 84 69.5) (end 84 65.75) (width 0.2) (layer "F.Cu") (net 9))
 (segment (start 84 65.75) (end 85.3 64.45) (width 0.2) (layer "F.Cu") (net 9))
 (segment (start 113.75 74.5) (end 111.9125 74.5) (width 0.2) (layer "F.Cu") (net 9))
 (segment (start 116.16 67.01) (end 116.16 66.49) (width 0.2) (layer "F.Cu") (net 9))
 (segment (start 106.2975 53.9125) (end 103.46 56.75) (width 0.2) (layer "F.Cu") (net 4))
 (segment (start 103.46 58.18) (end 104.28 59) (width 0.2) (layer "F.Cu") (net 4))
 (segment (start 114 60) (end 114 62.5) (width 0.2) (layer "F.Cu") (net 4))
 (segment (start 111.959448 62.75) (end 110.6 64.109448) (width 0.2) (layer "F.Cu") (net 4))
 (segment (start 110.6 71.4) (end 109.9125 72.0875) (width 0.2) (layer "F.Cu") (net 4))
 (segment (start 113 59) (end 114 60) (width 0.2) (layer "F.Cu") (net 4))
 (segment (start 103.46 57.725) (end 103.46 58.18) (width 0.2) (layer "F.Cu") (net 4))
 (segment (start 109.9125 72.0875) (end 92.5 72.0875) (width 0.2) (layer "F.Cu") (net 4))
 (segment (start 113.75 62.75) (end 111.959448 62.75) (width 0.2) (layer "F.Cu") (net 4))
 (segment (start 113.5 53.9125) (end 106.2975 53.9125) (width 0.2) (layer "F.Cu") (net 4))
 (segment (start 114 62.5) (end 113.75 62.75) (width 0.2) (layer "F.Cu") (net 4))
 (segment (start 103.46 56.75) (end 103.46 57.725) (width 0.2) (layer "F.Cu") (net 4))
 (segment (start 110.6 64.109448) (end 110.6 71.4) (width 0.2) (layer "F.Cu") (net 4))
 (segment (start 104.28 59) (end 113 59) (width 0.2) (layer "F.Cu") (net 4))
 (segment (start 111.2 73.3875) (end 110.0875 74.5) (width 0.2) (layer "F.Cu") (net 23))
 (segment (start 113.439339 64) (end 114.189339 63.25) (width 0.2) (layer "F.Cu") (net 23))
 (segment (start 118.7 64.395198) (end 118.7 65.47) (width 0.2) (layer "F.Cu") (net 23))
 (segment (start 114.189339 63.25) (end 117.554802 63.25) (width 0.2) (layer "F.Cu") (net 23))
 (segment (start 111.2 70.5) (end 111.2 73.3875) (width 0.2) (layer "F.Cu") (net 23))
 (segment (start 111.2 70.5) (end 111.2 67.5) (width 0.2) (layer "F.Cu") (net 23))
 (segment (start 117.554802 63.25) (end 118.7 64.395198) (width 0.2) (layer "F.Cu") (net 23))
 (segment (start 111.7 64) (end 113.439339 64) (width 0.2) (layer "F.Cu") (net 23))
 (segment (start 111.2 67.5) (end 111.2 64.5) (width 0.2) (layer "F.Cu") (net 23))
 (segment (start 111.2 64.5) (end 111.7 64) (width 0.2) (layer "F.Cu") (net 23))
 (segment (start 106.81 64.46) (end 109.76 64.46) (width 0.2) (layer "F.Cu") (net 30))
 (segment (start 109.76 64.46) (end 109.8 64.5) (width 0.2) (layer "F.Cu") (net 30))
 (segment (start 106.81 69.54) (end 108.84 69.54) (width 0.2) (layer "F.Cu") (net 24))
 (segment (start 108.84 69.54) (end 109.8 70.5) (width 0.2) (layer "F.Cu") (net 24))
 (segment (start 91 63.5) (end 92 62.5) (width 0.2) (layer "F.Cu") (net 17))
 (segment (start 87.84 69.55) (end 88.8 69.55) (width 0.2) (layer "F.Cu") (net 17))
 (segment (start 92 62.5) (end 97.23 62.5) (width 0.2) (layer "F.Cu") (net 17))
 (segment (start 116.16 64.45) (end 114.95 64.45) (width 0.2) (layer "F.Cu") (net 17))
 (segment (start 99.19 63.31) (end 99.19 64.46) (width 0.2) (layer "F.Cu") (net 17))
 (segment (start 97.23 62.5) (end 99.19 64.46) (width 0.2) (layer "F.Cu") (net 17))
 (segment (start 91 67.35) (end 91 63.5) (width 0.2) (layer "F.Cu") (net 17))
 (segment (start 88.8 69.55) (end 91 67.35) (width 0.2) (layer "F.Cu") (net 17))
 (segment (start 114.95 64.45) (end 114.5 64) (width 0.2) (layer "F.Cu") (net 17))
 (segment (start 100 62.5) (end 99.19 63.31) (width 0.2) (layer "F.Cu") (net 17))
 (via (at 100 62.5) (size 0.9) (drill 0.4) (layers "F.Cu" "B.Cu") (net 17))
 (via (at 114.5 64) (size 0.9) (drill 0.4) (layers "F.Cu" "B.Cu") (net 17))
 (segment (start 101.25 61.25) (end 100 62.5) (width 0.2) (layer "B.Cu") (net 17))
 (segment (start 114.5 62.939339) (end 112.810661 61.25) (width 0.2) (layer "B.Cu") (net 17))
 (segment (start 114.5 64) (end 114.5 62.939339) (width 0.2) (layer "B.Cu") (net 17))
 (segment (start 112.810661 61.25) (end 101.25 61.25) (width 0.2) (layer "B.Cu") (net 17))
 (segment (start 85.3 69.3) (end 85.3 68.53) (width 0.2) (layer "F.Cu") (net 18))
 (segment (start 95.978052 67) (end 93.770209 69.207843) (width 0.2) (layer "F.Cu") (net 18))
 (segment (start 89 71) (end 87 71) (width 0.2) (layer "F.Cu") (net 18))
 (segment (start 87 71) (end 85.3 69.3) (width 0.2) (layer "F.Cu") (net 18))
 (segment (start 93.770209 69.207843) (end 90.792157 69.207843) (width 0.2) (layer "F.Cu") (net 18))
 (segment (start 90.792157 69.207843) (end 89 71) (width 0.2) (layer "F.Cu") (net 18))
 (segment (start 99.19 67) (end 95.978052 67) (width 0.2) (layer "F.Cu") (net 18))
 (segment (start 87.84 59.375) (end 87.84 65.47) (width 0.2) (layer "F.Cu") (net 20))
 (segment (start 85.735 57.27) (end 87.84 59.375) (width 0.2) (layer "F.Cu") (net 20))
 (segment (start 111.9125 50.5) (end 102.035 50.5) (width 0.2) (layer "F.Cu") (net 25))
 (segment (start 113.5 52.0875) (end 111.9125 50.5) (width 0.2) (layer "F.Cu") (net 25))
 (segment (start 102.035 50.5) (end 95.265 57.27) (width 0.2) (layer "F.Cu") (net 25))
 (segment (start 106.81 67) (end 109.3 67) (width 0.2) (layer "F.Cu") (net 29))
 (segment (start 109.3 67) (end 109.8 67.5) (width 0.2) (layer "F.Cu") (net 29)))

